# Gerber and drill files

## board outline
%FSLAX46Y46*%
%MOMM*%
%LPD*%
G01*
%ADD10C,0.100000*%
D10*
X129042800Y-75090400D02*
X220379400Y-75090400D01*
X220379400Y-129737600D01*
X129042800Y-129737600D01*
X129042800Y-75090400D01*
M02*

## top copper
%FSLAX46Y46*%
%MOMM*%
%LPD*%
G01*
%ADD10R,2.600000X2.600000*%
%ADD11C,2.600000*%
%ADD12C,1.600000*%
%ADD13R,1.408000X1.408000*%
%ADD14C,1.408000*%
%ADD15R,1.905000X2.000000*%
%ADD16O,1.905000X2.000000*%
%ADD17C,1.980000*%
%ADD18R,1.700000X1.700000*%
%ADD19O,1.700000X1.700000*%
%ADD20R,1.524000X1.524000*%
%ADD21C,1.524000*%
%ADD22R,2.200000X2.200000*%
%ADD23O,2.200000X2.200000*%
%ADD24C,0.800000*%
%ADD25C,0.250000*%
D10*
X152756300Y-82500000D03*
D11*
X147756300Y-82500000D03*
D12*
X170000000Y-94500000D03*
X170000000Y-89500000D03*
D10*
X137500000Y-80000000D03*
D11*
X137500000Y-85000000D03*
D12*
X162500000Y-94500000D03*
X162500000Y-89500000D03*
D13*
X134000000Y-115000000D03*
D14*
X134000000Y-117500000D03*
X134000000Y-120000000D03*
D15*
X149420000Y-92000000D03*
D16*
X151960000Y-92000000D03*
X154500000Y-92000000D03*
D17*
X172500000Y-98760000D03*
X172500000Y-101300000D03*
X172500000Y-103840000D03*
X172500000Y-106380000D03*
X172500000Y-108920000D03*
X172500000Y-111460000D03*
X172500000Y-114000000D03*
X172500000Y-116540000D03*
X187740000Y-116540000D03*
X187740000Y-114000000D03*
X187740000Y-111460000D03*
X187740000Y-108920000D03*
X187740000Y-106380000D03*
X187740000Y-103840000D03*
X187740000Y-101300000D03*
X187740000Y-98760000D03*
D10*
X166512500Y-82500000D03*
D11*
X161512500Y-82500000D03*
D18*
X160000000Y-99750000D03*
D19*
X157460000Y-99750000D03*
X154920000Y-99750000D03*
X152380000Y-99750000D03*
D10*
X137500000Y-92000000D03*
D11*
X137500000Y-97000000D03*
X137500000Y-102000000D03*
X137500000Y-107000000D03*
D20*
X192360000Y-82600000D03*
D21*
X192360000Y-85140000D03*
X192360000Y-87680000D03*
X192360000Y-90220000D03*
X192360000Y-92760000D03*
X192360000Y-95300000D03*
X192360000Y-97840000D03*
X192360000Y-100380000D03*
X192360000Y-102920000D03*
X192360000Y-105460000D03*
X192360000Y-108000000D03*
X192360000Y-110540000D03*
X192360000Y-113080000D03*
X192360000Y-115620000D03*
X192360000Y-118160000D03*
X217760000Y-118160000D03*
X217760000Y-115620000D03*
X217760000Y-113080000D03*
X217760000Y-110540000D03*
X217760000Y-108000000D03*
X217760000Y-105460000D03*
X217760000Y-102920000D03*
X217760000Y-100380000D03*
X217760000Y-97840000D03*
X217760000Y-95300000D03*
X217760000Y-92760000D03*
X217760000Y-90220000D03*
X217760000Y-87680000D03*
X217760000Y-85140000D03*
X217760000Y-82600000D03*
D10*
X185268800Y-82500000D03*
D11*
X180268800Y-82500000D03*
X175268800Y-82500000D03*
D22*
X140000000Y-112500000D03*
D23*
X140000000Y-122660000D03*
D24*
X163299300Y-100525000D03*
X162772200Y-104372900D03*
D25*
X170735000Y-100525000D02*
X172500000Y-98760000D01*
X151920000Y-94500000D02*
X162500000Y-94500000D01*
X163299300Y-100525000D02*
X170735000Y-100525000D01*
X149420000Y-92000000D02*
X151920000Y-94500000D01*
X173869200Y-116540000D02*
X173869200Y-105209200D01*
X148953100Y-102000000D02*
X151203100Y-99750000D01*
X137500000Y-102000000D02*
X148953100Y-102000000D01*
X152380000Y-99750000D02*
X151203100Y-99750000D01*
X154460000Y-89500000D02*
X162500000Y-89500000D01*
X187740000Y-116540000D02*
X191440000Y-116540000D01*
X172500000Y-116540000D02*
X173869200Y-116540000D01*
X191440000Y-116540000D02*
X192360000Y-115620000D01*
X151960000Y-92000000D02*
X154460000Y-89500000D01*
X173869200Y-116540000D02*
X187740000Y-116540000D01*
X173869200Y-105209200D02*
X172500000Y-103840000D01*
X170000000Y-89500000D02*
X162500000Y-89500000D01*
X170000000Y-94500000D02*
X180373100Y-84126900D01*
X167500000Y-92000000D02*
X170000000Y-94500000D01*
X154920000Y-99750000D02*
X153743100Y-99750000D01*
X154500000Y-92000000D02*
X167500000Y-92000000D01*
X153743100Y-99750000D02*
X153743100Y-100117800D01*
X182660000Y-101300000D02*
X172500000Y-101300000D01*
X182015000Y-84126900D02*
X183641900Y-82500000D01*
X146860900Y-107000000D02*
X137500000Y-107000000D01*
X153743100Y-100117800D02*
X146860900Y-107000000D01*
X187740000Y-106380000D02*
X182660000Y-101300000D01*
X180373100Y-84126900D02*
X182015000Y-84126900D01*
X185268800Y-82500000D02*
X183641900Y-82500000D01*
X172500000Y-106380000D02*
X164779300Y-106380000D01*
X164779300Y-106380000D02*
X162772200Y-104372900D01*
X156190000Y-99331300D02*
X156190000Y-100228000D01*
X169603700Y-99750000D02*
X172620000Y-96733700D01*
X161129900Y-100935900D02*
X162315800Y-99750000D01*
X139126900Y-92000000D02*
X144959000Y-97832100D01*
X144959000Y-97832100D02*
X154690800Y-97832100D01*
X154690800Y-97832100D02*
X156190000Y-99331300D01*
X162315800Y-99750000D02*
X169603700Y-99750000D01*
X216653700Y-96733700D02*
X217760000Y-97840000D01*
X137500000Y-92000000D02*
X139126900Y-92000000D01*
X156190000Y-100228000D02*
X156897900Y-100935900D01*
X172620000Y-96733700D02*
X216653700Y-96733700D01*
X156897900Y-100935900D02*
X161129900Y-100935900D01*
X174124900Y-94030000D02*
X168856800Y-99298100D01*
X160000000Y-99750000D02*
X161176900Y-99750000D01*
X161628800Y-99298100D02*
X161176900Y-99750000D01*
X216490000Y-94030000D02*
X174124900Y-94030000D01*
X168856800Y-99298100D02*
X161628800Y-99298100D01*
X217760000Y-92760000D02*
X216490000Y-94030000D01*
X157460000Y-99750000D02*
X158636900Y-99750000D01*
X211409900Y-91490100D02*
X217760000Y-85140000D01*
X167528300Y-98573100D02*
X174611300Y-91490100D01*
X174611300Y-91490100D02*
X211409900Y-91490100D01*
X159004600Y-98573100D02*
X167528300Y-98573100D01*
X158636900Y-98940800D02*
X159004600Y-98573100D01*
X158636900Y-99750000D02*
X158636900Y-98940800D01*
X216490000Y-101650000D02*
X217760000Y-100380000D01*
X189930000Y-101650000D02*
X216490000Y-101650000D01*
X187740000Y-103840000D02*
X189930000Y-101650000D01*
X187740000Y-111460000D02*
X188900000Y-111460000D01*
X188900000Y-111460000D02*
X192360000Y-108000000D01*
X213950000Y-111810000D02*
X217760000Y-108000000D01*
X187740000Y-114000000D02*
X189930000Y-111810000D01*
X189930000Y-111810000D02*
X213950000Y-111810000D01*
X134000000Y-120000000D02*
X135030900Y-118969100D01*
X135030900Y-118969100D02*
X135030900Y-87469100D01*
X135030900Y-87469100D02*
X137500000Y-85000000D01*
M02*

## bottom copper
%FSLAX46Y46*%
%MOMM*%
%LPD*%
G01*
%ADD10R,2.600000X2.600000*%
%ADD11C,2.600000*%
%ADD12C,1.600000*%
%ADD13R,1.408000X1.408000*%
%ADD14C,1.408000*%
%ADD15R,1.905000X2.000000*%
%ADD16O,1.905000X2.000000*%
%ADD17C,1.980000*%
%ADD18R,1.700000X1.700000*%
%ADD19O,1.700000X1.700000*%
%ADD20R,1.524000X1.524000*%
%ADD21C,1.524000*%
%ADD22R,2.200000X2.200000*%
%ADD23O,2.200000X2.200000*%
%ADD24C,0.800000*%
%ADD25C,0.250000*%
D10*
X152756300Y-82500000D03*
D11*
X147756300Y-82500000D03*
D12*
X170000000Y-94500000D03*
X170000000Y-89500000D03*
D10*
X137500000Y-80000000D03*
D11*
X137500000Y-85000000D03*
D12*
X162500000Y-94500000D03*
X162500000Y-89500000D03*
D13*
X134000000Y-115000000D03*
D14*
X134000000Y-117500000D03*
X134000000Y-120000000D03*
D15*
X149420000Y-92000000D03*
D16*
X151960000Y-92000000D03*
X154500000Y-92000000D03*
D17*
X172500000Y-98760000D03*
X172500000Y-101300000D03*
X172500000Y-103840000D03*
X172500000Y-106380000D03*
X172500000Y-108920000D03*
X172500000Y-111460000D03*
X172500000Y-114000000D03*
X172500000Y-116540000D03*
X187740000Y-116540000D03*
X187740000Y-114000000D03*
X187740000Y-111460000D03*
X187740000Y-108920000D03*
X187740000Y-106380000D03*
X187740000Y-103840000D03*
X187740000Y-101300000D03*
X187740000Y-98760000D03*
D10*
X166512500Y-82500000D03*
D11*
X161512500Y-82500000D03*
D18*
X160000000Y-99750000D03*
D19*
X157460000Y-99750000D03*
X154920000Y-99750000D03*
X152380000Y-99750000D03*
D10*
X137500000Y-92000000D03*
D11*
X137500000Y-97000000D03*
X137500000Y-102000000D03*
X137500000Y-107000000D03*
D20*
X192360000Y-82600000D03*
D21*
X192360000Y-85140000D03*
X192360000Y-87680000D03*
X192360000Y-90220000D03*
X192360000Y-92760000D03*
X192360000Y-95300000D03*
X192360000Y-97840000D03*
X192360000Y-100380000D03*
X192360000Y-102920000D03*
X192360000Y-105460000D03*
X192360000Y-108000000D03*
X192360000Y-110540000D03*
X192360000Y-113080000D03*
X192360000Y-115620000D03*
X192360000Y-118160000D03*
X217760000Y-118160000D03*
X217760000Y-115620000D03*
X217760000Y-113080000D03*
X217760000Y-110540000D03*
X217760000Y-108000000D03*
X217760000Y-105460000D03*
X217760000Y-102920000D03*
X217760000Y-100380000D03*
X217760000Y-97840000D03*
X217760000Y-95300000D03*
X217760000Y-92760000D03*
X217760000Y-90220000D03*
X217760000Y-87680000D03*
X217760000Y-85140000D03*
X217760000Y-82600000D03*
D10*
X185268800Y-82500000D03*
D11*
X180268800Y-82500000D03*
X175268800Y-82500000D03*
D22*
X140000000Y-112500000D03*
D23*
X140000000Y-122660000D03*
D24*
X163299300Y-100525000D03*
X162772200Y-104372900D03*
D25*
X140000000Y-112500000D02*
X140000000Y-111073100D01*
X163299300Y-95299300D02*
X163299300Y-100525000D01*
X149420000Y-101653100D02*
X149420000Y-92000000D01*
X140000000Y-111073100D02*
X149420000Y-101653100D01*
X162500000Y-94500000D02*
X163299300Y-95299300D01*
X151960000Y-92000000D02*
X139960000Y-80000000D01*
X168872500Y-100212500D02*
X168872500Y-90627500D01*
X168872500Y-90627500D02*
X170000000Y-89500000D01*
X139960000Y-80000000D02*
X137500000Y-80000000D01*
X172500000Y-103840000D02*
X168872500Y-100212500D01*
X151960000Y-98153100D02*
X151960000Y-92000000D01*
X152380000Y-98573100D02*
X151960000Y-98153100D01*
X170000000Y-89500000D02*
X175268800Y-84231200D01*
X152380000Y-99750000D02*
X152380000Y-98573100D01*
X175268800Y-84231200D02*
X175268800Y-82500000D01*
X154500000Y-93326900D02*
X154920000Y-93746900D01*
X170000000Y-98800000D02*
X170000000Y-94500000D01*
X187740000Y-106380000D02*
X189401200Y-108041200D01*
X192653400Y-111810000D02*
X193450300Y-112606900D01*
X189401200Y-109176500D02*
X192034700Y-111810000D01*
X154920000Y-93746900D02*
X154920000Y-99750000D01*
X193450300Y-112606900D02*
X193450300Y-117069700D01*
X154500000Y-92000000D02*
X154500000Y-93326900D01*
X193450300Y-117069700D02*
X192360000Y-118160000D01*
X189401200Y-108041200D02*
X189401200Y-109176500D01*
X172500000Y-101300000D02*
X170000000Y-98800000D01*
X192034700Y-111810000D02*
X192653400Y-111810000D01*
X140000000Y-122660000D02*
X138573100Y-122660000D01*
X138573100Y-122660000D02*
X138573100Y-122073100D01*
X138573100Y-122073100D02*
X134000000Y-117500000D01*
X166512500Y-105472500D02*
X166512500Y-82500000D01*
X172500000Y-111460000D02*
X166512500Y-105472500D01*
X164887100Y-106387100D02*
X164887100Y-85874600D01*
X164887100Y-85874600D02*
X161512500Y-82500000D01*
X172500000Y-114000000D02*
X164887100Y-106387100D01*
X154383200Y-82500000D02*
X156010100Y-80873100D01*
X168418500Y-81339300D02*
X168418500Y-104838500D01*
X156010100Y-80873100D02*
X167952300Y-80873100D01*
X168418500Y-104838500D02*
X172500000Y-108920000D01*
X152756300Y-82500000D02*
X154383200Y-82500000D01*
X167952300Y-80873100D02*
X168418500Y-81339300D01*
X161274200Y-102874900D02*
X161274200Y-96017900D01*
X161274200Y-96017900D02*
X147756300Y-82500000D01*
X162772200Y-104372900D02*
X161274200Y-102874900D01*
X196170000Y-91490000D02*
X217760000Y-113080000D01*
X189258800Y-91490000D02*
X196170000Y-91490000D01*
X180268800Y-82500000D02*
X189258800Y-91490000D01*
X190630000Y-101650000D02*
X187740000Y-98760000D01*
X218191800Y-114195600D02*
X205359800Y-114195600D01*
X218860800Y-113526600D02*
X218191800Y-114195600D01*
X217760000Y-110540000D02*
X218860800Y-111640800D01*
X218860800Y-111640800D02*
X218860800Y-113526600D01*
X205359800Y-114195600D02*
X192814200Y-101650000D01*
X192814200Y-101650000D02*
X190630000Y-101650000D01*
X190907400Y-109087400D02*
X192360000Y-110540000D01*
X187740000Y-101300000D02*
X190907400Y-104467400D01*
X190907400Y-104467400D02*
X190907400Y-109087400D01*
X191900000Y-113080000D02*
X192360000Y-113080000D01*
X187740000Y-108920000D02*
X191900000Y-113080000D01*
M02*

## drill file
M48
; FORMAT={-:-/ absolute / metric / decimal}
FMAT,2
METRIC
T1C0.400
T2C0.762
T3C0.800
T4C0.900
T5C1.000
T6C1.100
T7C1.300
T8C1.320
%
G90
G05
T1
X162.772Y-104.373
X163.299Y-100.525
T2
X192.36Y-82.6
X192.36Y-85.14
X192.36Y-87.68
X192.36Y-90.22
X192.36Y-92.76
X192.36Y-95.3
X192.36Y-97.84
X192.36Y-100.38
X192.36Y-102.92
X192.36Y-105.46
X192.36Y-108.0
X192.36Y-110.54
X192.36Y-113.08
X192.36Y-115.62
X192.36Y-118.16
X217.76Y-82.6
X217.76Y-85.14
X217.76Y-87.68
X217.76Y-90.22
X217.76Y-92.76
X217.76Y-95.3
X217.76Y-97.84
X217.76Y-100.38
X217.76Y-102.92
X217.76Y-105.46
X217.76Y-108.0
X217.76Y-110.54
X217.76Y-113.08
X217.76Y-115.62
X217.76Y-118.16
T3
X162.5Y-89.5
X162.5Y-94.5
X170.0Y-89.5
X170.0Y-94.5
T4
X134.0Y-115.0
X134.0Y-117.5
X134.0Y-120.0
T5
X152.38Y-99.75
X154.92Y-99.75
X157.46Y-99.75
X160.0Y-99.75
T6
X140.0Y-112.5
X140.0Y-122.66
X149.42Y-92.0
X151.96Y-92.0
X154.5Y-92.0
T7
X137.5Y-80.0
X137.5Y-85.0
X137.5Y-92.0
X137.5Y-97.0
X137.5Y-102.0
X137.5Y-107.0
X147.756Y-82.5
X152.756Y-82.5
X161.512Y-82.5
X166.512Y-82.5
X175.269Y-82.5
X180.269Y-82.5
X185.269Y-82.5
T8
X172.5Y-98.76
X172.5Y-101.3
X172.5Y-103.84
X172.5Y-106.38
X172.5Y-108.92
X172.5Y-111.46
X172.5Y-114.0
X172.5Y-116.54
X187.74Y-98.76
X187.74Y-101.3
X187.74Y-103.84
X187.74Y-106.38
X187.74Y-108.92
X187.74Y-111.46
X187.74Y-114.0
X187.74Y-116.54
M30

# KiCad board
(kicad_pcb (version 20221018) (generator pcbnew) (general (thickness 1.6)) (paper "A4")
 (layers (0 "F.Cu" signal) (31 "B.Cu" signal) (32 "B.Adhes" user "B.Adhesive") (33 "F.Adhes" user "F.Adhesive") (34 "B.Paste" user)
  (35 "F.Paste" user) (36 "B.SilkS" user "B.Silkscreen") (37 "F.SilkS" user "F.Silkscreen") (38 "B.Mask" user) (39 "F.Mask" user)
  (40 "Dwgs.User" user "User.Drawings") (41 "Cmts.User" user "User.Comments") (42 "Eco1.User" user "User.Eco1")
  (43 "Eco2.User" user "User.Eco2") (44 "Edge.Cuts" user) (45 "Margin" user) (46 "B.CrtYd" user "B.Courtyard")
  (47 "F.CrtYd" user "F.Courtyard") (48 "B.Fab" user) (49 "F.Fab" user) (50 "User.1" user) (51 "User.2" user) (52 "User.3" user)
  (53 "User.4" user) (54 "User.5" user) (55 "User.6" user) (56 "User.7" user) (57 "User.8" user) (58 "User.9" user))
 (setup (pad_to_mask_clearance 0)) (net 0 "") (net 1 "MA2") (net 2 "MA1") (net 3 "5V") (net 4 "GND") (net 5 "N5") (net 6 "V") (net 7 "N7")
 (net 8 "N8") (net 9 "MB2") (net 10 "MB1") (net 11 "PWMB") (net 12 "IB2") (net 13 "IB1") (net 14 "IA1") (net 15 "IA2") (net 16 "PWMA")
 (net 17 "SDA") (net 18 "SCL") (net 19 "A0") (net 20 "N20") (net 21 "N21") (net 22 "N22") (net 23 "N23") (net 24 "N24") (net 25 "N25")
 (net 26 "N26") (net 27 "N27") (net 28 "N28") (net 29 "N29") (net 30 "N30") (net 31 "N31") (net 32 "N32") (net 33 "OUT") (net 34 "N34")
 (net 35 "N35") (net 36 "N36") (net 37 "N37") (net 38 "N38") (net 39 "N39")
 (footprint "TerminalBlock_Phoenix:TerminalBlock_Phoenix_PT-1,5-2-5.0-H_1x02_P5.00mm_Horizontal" (layer "F.Cu") (at 152.7563 82.5 180)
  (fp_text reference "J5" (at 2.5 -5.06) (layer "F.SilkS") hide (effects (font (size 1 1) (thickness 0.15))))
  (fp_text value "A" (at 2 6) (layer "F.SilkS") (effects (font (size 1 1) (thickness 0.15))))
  (pad "1" thru_hole rect (at 0 0 180) (size 2.6 2.6) (drill 1.3) (layers "*.Cu" "*.Mask") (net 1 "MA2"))
  (pad "2" thru_hole circle (at 5 0 180) (size 2.6 2.6) (drill 1.3) (layers "*.Cu" "*.Mask") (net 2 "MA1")))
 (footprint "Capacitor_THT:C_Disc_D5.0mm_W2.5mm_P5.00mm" (layer "F.Cu") (at 170 94.5 90)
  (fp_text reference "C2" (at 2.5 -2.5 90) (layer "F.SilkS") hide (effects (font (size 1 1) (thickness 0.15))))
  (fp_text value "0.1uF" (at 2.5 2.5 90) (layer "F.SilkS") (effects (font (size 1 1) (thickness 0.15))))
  (pad "1" thru_hole circle (at 0 0 90) (size 1.6 1.6) (drill 0.8) (layers "*.Cu" "*.Mask") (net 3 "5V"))
  (pad "2" thru_hole circle (at 5 0 90) (size 1.6 1.6) (drill 0.8) (layers "*.Cu" "*.Mask") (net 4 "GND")))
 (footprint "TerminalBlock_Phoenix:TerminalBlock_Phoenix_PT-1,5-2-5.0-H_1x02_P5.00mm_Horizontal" (layer "F.Cu") (at 137.5 80 -90)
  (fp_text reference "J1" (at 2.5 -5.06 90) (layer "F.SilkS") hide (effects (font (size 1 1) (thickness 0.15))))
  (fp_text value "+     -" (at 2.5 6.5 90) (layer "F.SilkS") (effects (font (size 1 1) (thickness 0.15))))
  (pad "1" thru_hole rect (at 0 0 270) (size 2.6 2.6) (drill 1.3) (layers "*.Cu" "*.Mask") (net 4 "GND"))
  (pad "2" thru_hole circle (at 5 0 270) (size 2.6 2.6) (drill 1.3) (layers "*.Cu" "*.Mask") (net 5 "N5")))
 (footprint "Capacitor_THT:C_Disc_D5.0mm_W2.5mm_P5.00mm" (layer "F.Cu") (at 162.5 94.5 90)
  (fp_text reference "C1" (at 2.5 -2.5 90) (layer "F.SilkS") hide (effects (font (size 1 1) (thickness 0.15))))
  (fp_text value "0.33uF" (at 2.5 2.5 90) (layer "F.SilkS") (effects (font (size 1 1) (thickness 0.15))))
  (pad "1" thru_hole circle (at 0 0 90) (size 1.6 1.6) (drill 0.8) (layers "*.Cu" "*.Mask") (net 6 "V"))
  (pad "2" thru_hole circle (at 5 0 90) (size 1.6 1.6) (drill 0.8) (layers "*.Cu" "*.Mask") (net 4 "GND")))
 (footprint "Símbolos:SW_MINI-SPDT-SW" (layer "F.Cu") (at 134 117.5 -90)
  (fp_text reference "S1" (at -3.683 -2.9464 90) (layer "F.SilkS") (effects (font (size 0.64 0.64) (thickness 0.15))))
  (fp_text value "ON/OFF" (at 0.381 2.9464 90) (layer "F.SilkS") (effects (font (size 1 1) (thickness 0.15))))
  (pad "1" thru_hole rect (at -2.5 0 270) (size 1.408 1.408) (drill 0.9) (layers "*.Cu" "*.Mask") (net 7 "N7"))
  (pad "2" thru_hole circle (at 0 0 270) (size 1.408 1.408) (drill 0.9) (layers "*.Cu" "*.Mask") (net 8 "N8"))
  (pad "3" thru_hole circle (at 2.5 0 270) (size 1.408 1.408) (drill 0.9) (layers "*.Cu" "*.Mask") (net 5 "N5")))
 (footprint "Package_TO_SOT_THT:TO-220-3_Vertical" (layer "F.Cu") (at 149.42 92)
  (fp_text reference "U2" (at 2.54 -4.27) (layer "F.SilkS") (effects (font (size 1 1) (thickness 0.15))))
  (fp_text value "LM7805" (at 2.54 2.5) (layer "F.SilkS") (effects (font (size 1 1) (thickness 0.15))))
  (pad "1" thru_hole rect (at 0 0) (size 1.905 2) (drill 1.1) (layers "*.Cu" "*.Mask") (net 6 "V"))
  (pad "2" thru_hole oval (at 2.54 0) (size 1.905 2) (drill 1.1) (layers "*.Cu" "*.Mask") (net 4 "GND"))
  (pad "3" thru_hole oval (at 5.08 0) (size 1.905 2) (drill 1.1) (layers "*.Cu" "*.Mask") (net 3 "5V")))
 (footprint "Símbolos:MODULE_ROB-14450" (layer "F.Cu") (at 180.12 107.65)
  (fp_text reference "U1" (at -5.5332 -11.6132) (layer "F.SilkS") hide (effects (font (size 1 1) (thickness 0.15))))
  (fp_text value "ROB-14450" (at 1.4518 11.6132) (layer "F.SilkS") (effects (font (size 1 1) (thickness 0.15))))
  (pad "1" thru_hole circle (at -7.62 -8.89) (size 1.98 1.98) (drill 1.32) (layers "*.Cu" "*.Mask") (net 6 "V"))
  (pad "2" thru_hole circle (at -7.62 -6.35) (size 1.98 1.98) (drill 1.32) (layers "*.Cu" "*.Mask") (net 3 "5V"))
  (pad "3" thru_hole circle (at -7.62 -3.81) (size 1.98 1.98) (drill 1.32) (layers "*.Cu" "*.Mask") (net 4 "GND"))
  (pad "4" thru_hole circle (at -7.62 -1.27) (size 1.98 1.98) (drill 1.32) (layers "*.Cu" "*.Mask") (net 2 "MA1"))
  (pad "5" thru_hole circle (at -7.62 1.27) (size 1.98 1.98) (drill 1.32) (layers "*.Cu" "*.Mask") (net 1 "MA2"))
  (pad "6" thru_hole circle (at -7.62 3.81) (size 1.98 1.98) (drill 1.32) (layers "*.Cu" "*.Mask") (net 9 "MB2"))
  (pad "7" thru_hole circle (at -7.62 6.35) (size 1.98 1.98) (drill 1.32) (layers "*.Cu" "*.Mask") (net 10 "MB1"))
  (pad "8" thru_hole circle (at -7.62 8.89) (size 1.98 1.98) (drill 1.32) (layers "*.Cu" "*.Mask") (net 4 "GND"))
  (pad "9" thru_hole circle (at 7.62 8.89) (size 1.98 1.98) (drill 1.32) (layers "*.Cu" "*.Mask") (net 4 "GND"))
  (pad "10" thru_hole circle (at 7.62 6.35) (size 1.98 1.98) (drill 1.32) (layers "*.Cu" "*.Mask") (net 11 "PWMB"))
  (pad "11" thru_hole circle (at 7.62 3.81) (size 1.98 1.98) (drill 1.32) (layers "*.Cu" "*.Mask") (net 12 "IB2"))
  (pad "12" thru_hole circle (at 7.62 1.27) (size 1.98 1.98) (drill 1.32) (layers "*.Cu" "*.Mask") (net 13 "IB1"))
  (pad "13" thru_hole circle (at 7.62 -1.27) (size 1.98 1.98) (drill 1.32) (layers "*.Cu" "*.Mask") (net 3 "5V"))
  (pad "14" thru_hole circle (at 7.62 -3.81) (size 1.98 1.98) (drill 1.32) (layers "*.Cu" "*.Mask") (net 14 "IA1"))
  (pad "15" thru_hole circle (at 7.62 -6.35) (size 1.98 1.98) (drill 1.32) (layers "*.Cu" "*.Mask") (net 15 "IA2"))
  (pad "16" thru_hole circle (at 7.62 -8.89) (size 1.98 1.98) (drill 1.32) (layers "*.Cu" "*.Mask") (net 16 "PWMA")))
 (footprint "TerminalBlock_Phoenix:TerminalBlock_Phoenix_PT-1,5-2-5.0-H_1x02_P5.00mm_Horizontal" (layer "F.Cu") (at 166.5125 82.5 180)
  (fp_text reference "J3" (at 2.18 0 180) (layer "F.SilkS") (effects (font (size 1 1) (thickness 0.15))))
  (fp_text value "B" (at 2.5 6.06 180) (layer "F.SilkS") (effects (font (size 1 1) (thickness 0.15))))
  (pad "1" thru_hole rect (at 0 0 180) (size 2.6 2.6) (drill 1.3) (layers "*.Cu" "*.Mask") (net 9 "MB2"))
  (pad "2" thru_hole circle (at 5 0 180) (size 2.6 2.6) (drill 1.3) (layers "*.Cu" "*.Mask") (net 10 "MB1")))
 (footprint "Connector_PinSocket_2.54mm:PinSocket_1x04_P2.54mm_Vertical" (layer "F.Cu") (at 160 99.75 -90)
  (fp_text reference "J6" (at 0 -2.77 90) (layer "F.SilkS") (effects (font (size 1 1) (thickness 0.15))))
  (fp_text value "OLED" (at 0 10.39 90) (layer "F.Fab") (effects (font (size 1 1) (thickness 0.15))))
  (pad "1" thru_hole rect (at 0 0 270) (size 1.7 1.7) (drill 1) (layers "*.Cu" "*.Mask") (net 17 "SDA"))
  (pad "2" thru_hole oval (at 0 2.54 270) (size 1.7 1.7) (drill 1) (layers "*.Cu" "*.Mask") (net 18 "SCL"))
  (pad "3" thru_hole oval (at 0 5.08 270) (size 1.7 1.7) (drill 1) (layers "*.Cu" "*.Mask") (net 3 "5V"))
  (pad "4" thru_hole oval (at 0 7.62 270) (size 1.7 1.7) (drill 1) (layers "*.Cu" "*.Mask") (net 4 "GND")))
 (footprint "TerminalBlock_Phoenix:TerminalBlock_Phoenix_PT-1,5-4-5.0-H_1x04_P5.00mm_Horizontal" (layer "F.Cu") (at 137.5 92 -90)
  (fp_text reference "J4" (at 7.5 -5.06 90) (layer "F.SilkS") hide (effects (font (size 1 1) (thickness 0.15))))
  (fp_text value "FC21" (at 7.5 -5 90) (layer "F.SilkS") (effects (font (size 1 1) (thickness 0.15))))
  (pad "1" thru_hole rect (at 0 0 270) (size 2.6 2.6) (drill 1.3) (layers "*.Cu" "*.Mask") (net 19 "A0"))
  (pad "2" thru_hole circle (at 5 0 270) (size 2.6 2.6) (drill 1.3) (layers "*.Cu" "*.Mask") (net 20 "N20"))
  (pad "3" thru_hole circle (at 10 0 270) (size 2.6 2.6) (drill 1.3) (layers "*.Cu" "*.Mask") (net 4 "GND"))
  (pad "4" thru_hole circle (at 15 0 270) (size 2.6 2.6) (drill 1.3) (layers "*.Cu" "*.Mask") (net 3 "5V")))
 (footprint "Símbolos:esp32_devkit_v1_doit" (layer "F.Cu") (at 205.06 82.6)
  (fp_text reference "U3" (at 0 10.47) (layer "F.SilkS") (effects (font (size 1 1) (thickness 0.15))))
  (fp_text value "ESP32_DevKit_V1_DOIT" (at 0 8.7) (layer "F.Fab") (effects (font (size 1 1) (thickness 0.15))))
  (pad "1" thru_hole rect (at -12.7 0) (size 1.524 1.524) (drill 0.762) (layers "*.Cu" "*.Mask") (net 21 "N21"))
  (pad "2" thru_hole circle (at -12.7 2.54) (size 1.524 1.524) (drill 0.762) (layers "*.Cu" "*.Mask") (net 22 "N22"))
  (pad "3" thru_hole circle (at -12.7 5.08) (size 1.524 1.524) (drill 0.762) (layers "*.Cu" "*.Mask") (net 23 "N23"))
  (pad "4" thru_hole circle (at -12.7 7.62) (size 1.524 1.524) (drill 0.762) (layers "*.Cu" "*.Mask") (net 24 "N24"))
  (pad "5" thru_hole circle (at -12.7 10.16) (size 1.524 1.524) (drill 0.762) (layers "*.Cu" "*.Mask") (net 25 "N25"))
  (pad "6" thru_hole circle (at -12.7 12.7) (size 1.524 1.524) (drill 0.762) (layers "*.Cu" "*.Mask") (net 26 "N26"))
  (pad "7" thru_hole circle (at -12.7 15.24) (size 1.524 1.524) (drill 0.762) (layers "*.Cu" "*.Mask") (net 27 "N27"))
  (pad "8" thru_hole circle (at -12.7 17.78) (size 1.524 1.524) (drill 0.762) (layers "*.Cu" "*.Mask") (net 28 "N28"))
  (pad "9" thru_hole circle (at -12.7 20.32) (size 1.524 1.524) (drill 0.762) (layers "*.Cu" "*.Mask") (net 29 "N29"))
  (pad "10" thru_hole circle (at -12.7 22.86) (size 1.524 1.524) (drill 0.762) (layers "*.Cu" "*.Mask") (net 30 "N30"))
  (pad "11" thru_hole circle (at -12.7 25.4) (size 1.524 1.524) (drill 0.762) (layers "*.Cu" "*.Mask") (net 12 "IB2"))
  (pad "12" thru_hole circle (at -12.7 27.94) (size 1.524 1.524) (drill 0.762) (layers "*.Cu" "*.Mask") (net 15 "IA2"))
  (pad "13" thru_hole circle (at -12.7 30.48) (size 1.524 1.524) (drill 0.762) (layers "*.Cu" "*.Mask") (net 13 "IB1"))
  (pad "14" thru_hole circle (at -12.7 33.02) (size 1.524 1.524) (drill 0.762) (layers "*.Cu" "*.Mask") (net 4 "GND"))
  (pad "15" thru_hole circle (at -12.7 35.56) (size 1.524 1.524) (drill 0.762) (layers "*.Cu" "*.Mask") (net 3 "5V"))
  (pad "16" thru_hole circle (at 12.7 35.56) (size 1.524 1.524) (drill 0.762) (layers "*.Cu" "*.Mask") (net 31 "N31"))
  (pad "17" thru_hole circle (at 12.7 33.02) (size 1.524 1.524) (drill 0.762) (layers "*.Cu" "*.Mask") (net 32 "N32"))
  (pad "18" thru_hole circle (at 12.7 30.48) (size 1.524 1.524) (drill 0.762) (layers "*.Cu" "*.Mask") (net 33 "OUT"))
  (pad "19" thru_hole circle (at 12.7 27.94) (size 1.524 1.524) (drill 0.762) (layers "*.Cu" "*.Mask") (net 16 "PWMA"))
  (pad "20" thru_hole circle (at 12.7 25.4) (size 1.524 1.524) (drill 0.762) (layers "*.Cu" "*.Mask") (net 11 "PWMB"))
  (pad "21" thru_hole circle (at 12.7 22.86) (size 1.524 1.524) (drill 0.762) (layers "*.Cu" "*.Mask") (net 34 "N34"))
  (pad "22" thru_hole circle (at 12.7 20.32) (size 1.524 1.524) (drill 0.762) (layers "*.Cu" "*.Mask") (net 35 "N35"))
  (pad "23" thru_hole circle (at 12.7 17.78) (size 1.524 1.524) (drill 0.762) (layers "*.Cu" "*.Mask") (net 14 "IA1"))
  (pad "24" thru_hole circle (at 12.7 15.24) (size 1.524 1.524) (drill 0.762) (layers "*.Cu" "*.Mask") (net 19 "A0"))
  (pad "25" thru_hole circle (at 12.7 12.7) (size 1.524 1.524) (drill 0.762) (layers "*.Cu" "*.Mask") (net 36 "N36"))
  (pad "26" thru_hole circle (at 12.7 10.16) (size 1.524 1.524) (drill 0.762) (layers "*.Cu" "*.Mask") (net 17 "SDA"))
  (pad "27" thru_hole circle (at 12.7 7.62) (size 1.524 1.524) (drill 0.762) (layers "*.Cu" "*.Mask") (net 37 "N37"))
  (pad "28" thru_hole circle (at 12.7 5.08) (size 1.524 1.524) (drill 0.762) (layers "*.Cu" "*.Mask") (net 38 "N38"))
  (pad "29" thru_hole circle (at 12.7 2.54) (size 1.524 1.524) (drill 0.762) (layers "*.Cu" "*.Mask") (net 18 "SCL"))
  (pad "30" thru_hole circle (at 12.7 0) (size 1.524 1.524) (drill 0.762) (layers "*.Cu" "*.Mask") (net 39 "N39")))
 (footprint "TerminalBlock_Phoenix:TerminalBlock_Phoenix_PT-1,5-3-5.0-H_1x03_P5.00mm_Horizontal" (layer "F.Cu") (at 185.2688 82.5 180)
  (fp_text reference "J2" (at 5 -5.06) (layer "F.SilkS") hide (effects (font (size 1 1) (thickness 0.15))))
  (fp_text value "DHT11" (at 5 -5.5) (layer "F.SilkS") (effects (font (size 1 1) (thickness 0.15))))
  (pad "1" thru_hole rect (at 0 0 180) (size 2.6 2.6) (drill 1.3) (layers "*.Cu" "*.Mask") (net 3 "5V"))
  (pad "2" thru_hole circle (at 5 0 180) (size 2.6 2.6) (drill 1.3) (layers "*.Cu" "*.Mask") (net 33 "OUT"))
  (pad "3" thru_hole circle (at 10 0 180) (size 2.6 2.6) (drill 1.3) (layers "*.Cu" "*.Mask") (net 4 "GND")))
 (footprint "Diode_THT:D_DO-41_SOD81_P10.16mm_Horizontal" (layer "F.Cu") (at 140 112.5 -90)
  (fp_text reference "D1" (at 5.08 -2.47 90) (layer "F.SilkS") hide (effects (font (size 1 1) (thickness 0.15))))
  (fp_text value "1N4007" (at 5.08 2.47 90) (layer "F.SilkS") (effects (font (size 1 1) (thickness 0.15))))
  (pad "1" thru_hole rect (at 0 0 270) (size 2.2 2.2) (drill 1.1) (layers "*.Cu" "*.Mask") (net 6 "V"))
  (pad "2" thru_hole oval (at 10.16 0 270) (size 2.2 2.2) (drill 1.1) (layers "*.Cu" "*.Mask") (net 8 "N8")))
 (gr_rect (start 129.0428 75.0904) (end 220.3794 129.7376) (stroke (width 0.1) (type default)) (fill none) (layer "Edge.Cuts"))
 (segment (start 170.735 100.525) (end 172.5 98.76) (width 0.25) (layer "F.Cu") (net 6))
 (segment (start 151.92 94.5) (end 162.5 94.5) (width 0.25) (layer "F.Cu") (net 6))
 (segment (start 163.2993 100.525) (end 170.735 100.525) (width 0.25) (layer "F.Cu") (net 6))
 (segment (start 149.42 92) (end 151.92 94.5) (width 0.25) (layer "F.Cu") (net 6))
 (via (at 163.2993 100.525) (size 0.8) (drill 0.4) (layers "F.Cu" "B.Cu") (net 6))
 (segment (start 140 112.5) (end 140 111.0731) (width 0.25) (layer "B.Cu") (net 6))
 (segment (start 163.2993 95.2993) (end 163.2993 100.525) (width 0.25) (layer "B.Cu") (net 6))
 (segment (start 149.42 101.6531) (end 149.42 92) (width 0.25) (layer "B.Cu") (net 6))
 (segment (start 140 111.0731) (end 149.42 101.6531) (width 0.25) (layer "B.Cu") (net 6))
 (segment (start 162.5 94.5) (end 163.2993 95.2993) (width 0.25) (layer "B.Cu") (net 6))
 (segment (start 173.8692 116.54) (end 173.8692 105.2092) (width 0.25) (layer "F.Cu") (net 4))
 (segment (start 148.9531 102) (end 151.2031 99.75) (width 0.25) (layer "F.Cu") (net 4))
 (segment (start 137.5 102) (end 148.9531 102) (width 0.25) (layer "F.Cu") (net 4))
 (segment (start 152.38 99.75) (end 151.2031 99.75) (width 0.25) (layer "F.Cu") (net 4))
 (segment (start 154.46 89.5) (end 162.5 89.5) (width 0.25) (layer "F.Cu") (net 4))
 (segment (start 187.74 116.54) (end 191.44 116.54) (width 0.25) (layer "F.Cu") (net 4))
 (segment (start 172.5 116.54) (end 173.8692 116.54) (width 0.25) (layer "F.Cu") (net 4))
 (segment (start 191.44 116.54) (end 192.36 115.62) (width 0.25) (layer "F.Cu") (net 4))
 (segment (start 151.96 92) (end 154.46 89.5) (width 0.25) (layer "F.Cu") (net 4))
 (segment (start 173.8692 116.54) (end 187.74 116.54) (width 0.25) (layer "F.Cu") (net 4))
 (segment (start 173.8692 105.2092) (end 172.5 103.84) (width 0.25) (layer "F.Cu") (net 4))
 (segment (start 170 89.5) (end 162.5 89.5) (width 0.25) (layer "F.Cu") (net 4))
 (segment (start 151.96 92) (end 139.96 80) (width 0.25) (layer "B.Cu") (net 4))
 (segment (start 168.8725 100.2125) (end 168.8725 90.6275) (width 0.25) (layer "B.Cu") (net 4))
 (segment (start 168.8725 90.6275) (end 170 89.5) (width 0.25) (layer "B.Cu") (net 4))
 (segment (start 139.96 80) (end 137.5 80) (width 0.25) (layer "B.Cu") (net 4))
 (segment (start 172.5 103.84) (end 168.8725 100.2125) (width 0.25) (layer "B.Cu") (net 4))
 (segment (start 151.96 98.1531) (end 151.96 92) (width 0.25) (layer "B.Cu") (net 4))
 (segment (start 152.38 98.5731) (end 151.96 98.1531) (width 0.25) (layer "B.Cu") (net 4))
 (segment (start 170 89.5) (end 175.2688 84.2312) (width 0.25) (layer "B.Cu") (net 4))
 (segment (start 152.38 99.75) (end 152.38 98.5731) (width 0.25) (layer "B.Cu") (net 4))
 (segment (start 175.2688 84.2312) (end 175.2688 82.5) (width 0.25) (layer "B.Cu") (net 4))
 (segment (start 170 94.5) (end 180.3731 84.1269) (width 0.25) (layer "F.Cu") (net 3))
 (segment (start 167.5 92) (end 170 94.5) (width 0.25) (layer "F.Cu") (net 3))
 (segment (start 154.92 99.75) (end 153.7431 99.75) (width 0.25) (layer "F.Cu") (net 3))
 (segment (start 154.5 92) (end 167.5 92) (width 0.25) (layer "F.Cu") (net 3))
 (segment (start 153.7431 99.75) (end 153.7431 100.1178) (width 0.25) (layer "F.Cu") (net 3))
 (segment (start 182.66 101.3) (end 172.5 101.3) (width 0.25) (layer "F.Cu") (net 3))
 (segment (start 182.015 84.1269) (end 183.6419 82.5) (width 0.25) (layer "F.Cu") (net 3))
 (segment (start 146.8609 107) (end 137.5 107) (width 0.25) (layer "F.Cu") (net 3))
 (segment (start 153.7431 100.1178) (end 146.8609 107) (width 0.25) (layer "F.Cu") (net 3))
 (segment (start 187.74 106.38) (end 182.66 101.3) (width 0.25) (layer "F.Cu") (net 3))
 (segment (start 180.3731 84.1269) (end 182.015 84.1269) (width 0.25) (layer "F.Cu") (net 3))
 (segment (start 185.2688 82.5) (end 183.6419 82.5) (width 0.25) (layer "F.Cu") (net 3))
 (segment (start 154.5 93.3269) (end 154.92 93.7469) (width 0.25) (layer "B.Cu") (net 3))
 (segment (start 170 98.8) (end 170 94.5) (width 0.25) (layer "B.Cu") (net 3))
 (segment (start 187.74 106.38) (end 189.4012 108.0412) (width 0.25) (layer "B.Cu") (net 3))
 (segment (start 192.6534 111.81) (end 193.4503 112.6069) (width 0.25) (layer "B.Cu") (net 3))
 (segment (start 189.4012 109.1765) (end 192.0347 111.81) (width 0.25) (layer "B.Cu") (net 3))
 (segment (start 154.92 93.7469) (end 154.92 99.75) (width 0.25) (layer "B.Cu") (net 3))
 (segment (start 193.4503 112.6069) (end 193.4503 117.0697) (width 0.25) (layer "B.Cu") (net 3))
 (segment (start 154.5 92) (end 154.5 93.3269) (width 0.25) (layer "B.Cu") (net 3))
 (segment (start 193.4503 117.0697) (end 192.36 118.16) (width 0.25) (layer "B.Cu") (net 3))
 (segment (start 189.4012 108.0412) (end 189.4012 109.1765) (width 0.25) (layer "B.Cu") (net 3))
 (segment (start 172.5 101.3) (end 170 98.8) (width 0.25) (layer "B.Cu") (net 3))
 (segment (start 192.0347 111.81) (end 192.6534 111.81) (width 0.25) (layer "B.Cu") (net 3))
 (segment (start 140 122.66) (end 138.5731 122.66) (width 0.25) (layer "B.Cu") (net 8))
 (segment (start 138.5731 122.66) (end 138.5731 122.0731) (width 0.25) (layer "B.Cu") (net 8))
 (segment (start 138.5731 122.0731) (end 134 117.5) (width 0.25) (layer "B.Cu") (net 8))
 (segment (start 166.5125 105.4725) (end 166.5125 82.5) (width 0.25) (layer "B.Cu") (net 9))
 (segment (start 172.5 111.46) (end 166.5125 105.4725) (width 0.25) (layer "B.Cu") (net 9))
 (segment (start 164.8871 106.3871) (end 164.8871 85.8746) (width 0.25) (layer "B.Cu") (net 10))
 (segment (start 164.8871 85.8746) (end 161.5125 82.5) (width 0.25) (layer "B.Cu") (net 10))
 (segment (start 172.5 114) (end 164.8871 106.3871) (width 0.25) (layer "B.Cu") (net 10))
 (segment (start 154.3832 82.5) (end 156.0101 80.8731) (width 0.25) (layer "B.Cu") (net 1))
 (segment (start 168.4185 81.3393) (end 168.4185 104.8385) (width 0.25) (layer "B.Cu") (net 1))
 (segment (start 156.0101 80.8731) (end 167.9523 80.8731) (width 0.25) (layer "B.Cu") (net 1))
 (segment (start 168.4185 104.8385) (end 172.5 108.92) (width 0.25) (layer "B.Cu") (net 1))
 (segment (start 152.7563 82.5) (end 154.3832 82.5) (width 0.25) (layer "B.Cu") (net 1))
 (segment (start 167.9523 80.8731) (end 168.4185 81.3393) (width 0.25) (layer "B.Cu") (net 1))
 (segment (start 172.5 106.38) (end 164.7793 106.38) (width 0.25) (layer "F.Cu") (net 2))
 (segment (start 164.7793 106.38) (end 162.7722 104.3729) (width 0.25) (layer "F.Cu") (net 2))
 (via (at 162.7722 104.3729) (size 0.8) (drill 0.4) (layers "F.Cu" "B.Cu") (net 2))
 (segment (start 161.2742 102.8749) (end 161.2742 96.0179) (width 0.25) (layer "B.Cu") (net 2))
 (segment (start 161.2742 96.0179) (end 147.7563 82.5) (width 0.25) (layer "B.Cu") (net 2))
 (segment (start 162.7722 104.3729) (end 161.2742 102.8749) (width 0.25) (layer "B.Cu") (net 2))
 (segment (start 156.19 99.3313) (end 156.19 100.228) (width 0.25) (layer "F.Cu") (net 19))
 (segment (start 169.6037 99.75) (end 172.62 96.7337) (width 0.25) (layer "F.Cu") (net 19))
 (segment (start 161.1299 100.9359) (end 162.3158 99.75) (width 0.25) (layer "F.Cu") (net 19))
 (segment (start 139.1269 92) (end 144.959 97.8321) (width 0.25) (layer "F.Cu") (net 19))
 (segment (start 144.959 97.8321) (end 154.6908 97.8321) (width 0.25) (layer "F.Cu") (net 19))
 (segment (start 154.6908 97.8321) (end 156.19 99.3313) (width 0.25) (layer "F.Cu") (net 19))
 (segment (start 162.3158 99.75) (end 169.6037 99.75) (width 0.25) (layer "F.Cu") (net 19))
 (segment (start 216.6537 96.7337) (end 217.76 97.84) (width 0.25) (layer "F.Cu") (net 19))
 (segment (start 137.5 92) (end 139.1269 92) (width 0.25) (layer "F.Cu") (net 19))
 (segment (start 156.19 100.228) (end 156.8979 100.9359) (width 0.25) (layer "F.Cu") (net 19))
 (segment (start 172.62 96.7337) (end 216.6537 96.7337) (width 0.25) (layer "F.Cu") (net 19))
 (segment (start 156.8979 100.9359) (end 161.1299 100.9359) (width 0.25) (layer "F.Cu") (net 19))
 (segment (start 196.17 91.49) (end 217.76 113.08) (width 0.25) (layer "B.Cu") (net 33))
 (segment (start 189.2588 91.49) (end 196.17 91.49) (width 0.25) (layer "B.Cu") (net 33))
 (segment (start 180.2688 82.5) (end 189.2588 91.49) (width 0.25) (layer "B.Cu") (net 33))
 (segment (start 174.1249 94.03) (end 168.8568 99.2981) (width 0.25) (layer "F.Cu") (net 17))
 (segment (start 160 99.75) (end 161.1769 99.75) (width 0.25) (layer "F.Cu") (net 17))
 (segment (start 161.6288 99.2981) (end 161.1769 99.75) (width 0.25) (layer "F.Cu") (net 17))
 (segment (start 216.49 94.03) (end 174.1249 94.03) (width 0.25) (layer "F.Cu") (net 17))
 (segment (start 168.8568 99.2981) (end 161.6288 99.2981) (width 0.25) (layer "F.Cu") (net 17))
 (segment (start 217.76 92.76) (end 216.49 94.03) (width 0.25) (layer "F.Cu") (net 17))
 (segment (start 157.46 99.75) (end 158.6369 99.75) (width 0.25) (layer "F.Cu") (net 18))
 (segment (start 211.4099 91.4901) (end 217.76 85.14) (width 0.25) (layer "F.Cu") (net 18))
 (segment (start 167.5283 98.5731) (end 174.6113 91.4901) (width 0.25) (layer "F.Cu") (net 18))
 (segment (start 174.6113 91.4901) (end 211.4099 91.4901) (width 0.25) (layer "F.Cu") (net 18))
 (segment (start 159.0046 98.5731) (end 167.5283 98.5731) (width 0.25) (layer "F.Cu") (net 18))
 (segment (start 158.6369 98.9408) (end 159.0046 98.5731) (width 0.25) (layer "F.Cu") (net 18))
 (segment (start 158.6369 99.75) (end 158.6369 98.9408) (width 0.25) (layer "F.Cu") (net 18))
 (segment (start 190.63 101.65) (end 187.74 98.76) (width 0.25) (layer "B.Cu") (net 16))
 (segment (start 218.1918 114.1956) (end 205.3598 114.1956) (width 0.25) (layer "B.Cu") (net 16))
 (segment (start 218.8608 113.5266) (end 218.1918 114.1956) (width 0.25) (layer "B.Cu") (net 16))
 (segment (start 217.76 110.54) (end 218.8608 111.6408) (width 0.25) (layer "B.Cu") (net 16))
 (segment (start 218.8608 111.6408) (end 218.8608 113.5266) (width 0.25) (layer "B.Cu") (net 16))
 (segment (start 205.3598 114.1956) (end 192.8142 101.65) (width 0.25) (layer "B.Cu") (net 16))
 (segment (start 192.8142 101.65) (end 190.63 101.65) (width 0.25) (layer "B.Cu") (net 16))
 (segment (start 190.9074 109.0874) (end 192.36 110.54) (width 0.25) (layer "B.Cu") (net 15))
 (segment (start 187.74 101.3) (end 190.9074 104.4674) (width 0.25) (layer "B.Cu") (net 15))
 (segment (start 190.9074 104.4674) (end 190.9074 109.0874) (width 0.25) (layer "B.Cu") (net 15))
 (segment (start 216.49 101.65) (end 217.76 100.38) (width 0.25) (layer "F.Cu") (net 14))
 (segment (start 189.93 101.65) (end 216.49 101.65) (width 0.25) (layer "F.Cu") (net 14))
 (segment (start 187.74 103.84) (end 189.93 101.65) (width 0.25) (layer "F.Cu") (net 14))
 (segment (start 191.9 113.08) (end 192.36 113.08) (width 0.25) (layer "B.Cu") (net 13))
 (segment (start 187.74 108.92) (end 191.9 113.08) (width 0.25) (layer "B.Cu") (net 13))
 (segment (start 187.74 111.46) (end 188.9 111.46) (width 0.25) (layer "F.Cu") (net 12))
 (segment (start 188.9 111.46) (end 192.36 108) (width 0.25) (layer "F.Cu") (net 12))
 (segment (start 213.95 111.81) (end 217.76 108) (width 0.25) (layer "F.Cu") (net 11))
 (segment (start 187.74 114) (end 189.93 111.81) (width 0.25) (layer "F.Cu") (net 11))
 (segment (start 189.93 111.81) (end 213.95 111.81) (width 0.25) (layer "F.Cu") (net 11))
 (segment (start 134 120) (end 135.0309 118.9691) (width 0.25) (layer "F.Cu") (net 5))
 (segment (start 135.0309 118.9691) (end 135.0309 87.4691) (width 0.25) (layer "F.Cu") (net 5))
 (segment (start 135.0309 87.4691) (end 137.5 85) (width 0.25) (layer "F.Cu") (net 5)))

